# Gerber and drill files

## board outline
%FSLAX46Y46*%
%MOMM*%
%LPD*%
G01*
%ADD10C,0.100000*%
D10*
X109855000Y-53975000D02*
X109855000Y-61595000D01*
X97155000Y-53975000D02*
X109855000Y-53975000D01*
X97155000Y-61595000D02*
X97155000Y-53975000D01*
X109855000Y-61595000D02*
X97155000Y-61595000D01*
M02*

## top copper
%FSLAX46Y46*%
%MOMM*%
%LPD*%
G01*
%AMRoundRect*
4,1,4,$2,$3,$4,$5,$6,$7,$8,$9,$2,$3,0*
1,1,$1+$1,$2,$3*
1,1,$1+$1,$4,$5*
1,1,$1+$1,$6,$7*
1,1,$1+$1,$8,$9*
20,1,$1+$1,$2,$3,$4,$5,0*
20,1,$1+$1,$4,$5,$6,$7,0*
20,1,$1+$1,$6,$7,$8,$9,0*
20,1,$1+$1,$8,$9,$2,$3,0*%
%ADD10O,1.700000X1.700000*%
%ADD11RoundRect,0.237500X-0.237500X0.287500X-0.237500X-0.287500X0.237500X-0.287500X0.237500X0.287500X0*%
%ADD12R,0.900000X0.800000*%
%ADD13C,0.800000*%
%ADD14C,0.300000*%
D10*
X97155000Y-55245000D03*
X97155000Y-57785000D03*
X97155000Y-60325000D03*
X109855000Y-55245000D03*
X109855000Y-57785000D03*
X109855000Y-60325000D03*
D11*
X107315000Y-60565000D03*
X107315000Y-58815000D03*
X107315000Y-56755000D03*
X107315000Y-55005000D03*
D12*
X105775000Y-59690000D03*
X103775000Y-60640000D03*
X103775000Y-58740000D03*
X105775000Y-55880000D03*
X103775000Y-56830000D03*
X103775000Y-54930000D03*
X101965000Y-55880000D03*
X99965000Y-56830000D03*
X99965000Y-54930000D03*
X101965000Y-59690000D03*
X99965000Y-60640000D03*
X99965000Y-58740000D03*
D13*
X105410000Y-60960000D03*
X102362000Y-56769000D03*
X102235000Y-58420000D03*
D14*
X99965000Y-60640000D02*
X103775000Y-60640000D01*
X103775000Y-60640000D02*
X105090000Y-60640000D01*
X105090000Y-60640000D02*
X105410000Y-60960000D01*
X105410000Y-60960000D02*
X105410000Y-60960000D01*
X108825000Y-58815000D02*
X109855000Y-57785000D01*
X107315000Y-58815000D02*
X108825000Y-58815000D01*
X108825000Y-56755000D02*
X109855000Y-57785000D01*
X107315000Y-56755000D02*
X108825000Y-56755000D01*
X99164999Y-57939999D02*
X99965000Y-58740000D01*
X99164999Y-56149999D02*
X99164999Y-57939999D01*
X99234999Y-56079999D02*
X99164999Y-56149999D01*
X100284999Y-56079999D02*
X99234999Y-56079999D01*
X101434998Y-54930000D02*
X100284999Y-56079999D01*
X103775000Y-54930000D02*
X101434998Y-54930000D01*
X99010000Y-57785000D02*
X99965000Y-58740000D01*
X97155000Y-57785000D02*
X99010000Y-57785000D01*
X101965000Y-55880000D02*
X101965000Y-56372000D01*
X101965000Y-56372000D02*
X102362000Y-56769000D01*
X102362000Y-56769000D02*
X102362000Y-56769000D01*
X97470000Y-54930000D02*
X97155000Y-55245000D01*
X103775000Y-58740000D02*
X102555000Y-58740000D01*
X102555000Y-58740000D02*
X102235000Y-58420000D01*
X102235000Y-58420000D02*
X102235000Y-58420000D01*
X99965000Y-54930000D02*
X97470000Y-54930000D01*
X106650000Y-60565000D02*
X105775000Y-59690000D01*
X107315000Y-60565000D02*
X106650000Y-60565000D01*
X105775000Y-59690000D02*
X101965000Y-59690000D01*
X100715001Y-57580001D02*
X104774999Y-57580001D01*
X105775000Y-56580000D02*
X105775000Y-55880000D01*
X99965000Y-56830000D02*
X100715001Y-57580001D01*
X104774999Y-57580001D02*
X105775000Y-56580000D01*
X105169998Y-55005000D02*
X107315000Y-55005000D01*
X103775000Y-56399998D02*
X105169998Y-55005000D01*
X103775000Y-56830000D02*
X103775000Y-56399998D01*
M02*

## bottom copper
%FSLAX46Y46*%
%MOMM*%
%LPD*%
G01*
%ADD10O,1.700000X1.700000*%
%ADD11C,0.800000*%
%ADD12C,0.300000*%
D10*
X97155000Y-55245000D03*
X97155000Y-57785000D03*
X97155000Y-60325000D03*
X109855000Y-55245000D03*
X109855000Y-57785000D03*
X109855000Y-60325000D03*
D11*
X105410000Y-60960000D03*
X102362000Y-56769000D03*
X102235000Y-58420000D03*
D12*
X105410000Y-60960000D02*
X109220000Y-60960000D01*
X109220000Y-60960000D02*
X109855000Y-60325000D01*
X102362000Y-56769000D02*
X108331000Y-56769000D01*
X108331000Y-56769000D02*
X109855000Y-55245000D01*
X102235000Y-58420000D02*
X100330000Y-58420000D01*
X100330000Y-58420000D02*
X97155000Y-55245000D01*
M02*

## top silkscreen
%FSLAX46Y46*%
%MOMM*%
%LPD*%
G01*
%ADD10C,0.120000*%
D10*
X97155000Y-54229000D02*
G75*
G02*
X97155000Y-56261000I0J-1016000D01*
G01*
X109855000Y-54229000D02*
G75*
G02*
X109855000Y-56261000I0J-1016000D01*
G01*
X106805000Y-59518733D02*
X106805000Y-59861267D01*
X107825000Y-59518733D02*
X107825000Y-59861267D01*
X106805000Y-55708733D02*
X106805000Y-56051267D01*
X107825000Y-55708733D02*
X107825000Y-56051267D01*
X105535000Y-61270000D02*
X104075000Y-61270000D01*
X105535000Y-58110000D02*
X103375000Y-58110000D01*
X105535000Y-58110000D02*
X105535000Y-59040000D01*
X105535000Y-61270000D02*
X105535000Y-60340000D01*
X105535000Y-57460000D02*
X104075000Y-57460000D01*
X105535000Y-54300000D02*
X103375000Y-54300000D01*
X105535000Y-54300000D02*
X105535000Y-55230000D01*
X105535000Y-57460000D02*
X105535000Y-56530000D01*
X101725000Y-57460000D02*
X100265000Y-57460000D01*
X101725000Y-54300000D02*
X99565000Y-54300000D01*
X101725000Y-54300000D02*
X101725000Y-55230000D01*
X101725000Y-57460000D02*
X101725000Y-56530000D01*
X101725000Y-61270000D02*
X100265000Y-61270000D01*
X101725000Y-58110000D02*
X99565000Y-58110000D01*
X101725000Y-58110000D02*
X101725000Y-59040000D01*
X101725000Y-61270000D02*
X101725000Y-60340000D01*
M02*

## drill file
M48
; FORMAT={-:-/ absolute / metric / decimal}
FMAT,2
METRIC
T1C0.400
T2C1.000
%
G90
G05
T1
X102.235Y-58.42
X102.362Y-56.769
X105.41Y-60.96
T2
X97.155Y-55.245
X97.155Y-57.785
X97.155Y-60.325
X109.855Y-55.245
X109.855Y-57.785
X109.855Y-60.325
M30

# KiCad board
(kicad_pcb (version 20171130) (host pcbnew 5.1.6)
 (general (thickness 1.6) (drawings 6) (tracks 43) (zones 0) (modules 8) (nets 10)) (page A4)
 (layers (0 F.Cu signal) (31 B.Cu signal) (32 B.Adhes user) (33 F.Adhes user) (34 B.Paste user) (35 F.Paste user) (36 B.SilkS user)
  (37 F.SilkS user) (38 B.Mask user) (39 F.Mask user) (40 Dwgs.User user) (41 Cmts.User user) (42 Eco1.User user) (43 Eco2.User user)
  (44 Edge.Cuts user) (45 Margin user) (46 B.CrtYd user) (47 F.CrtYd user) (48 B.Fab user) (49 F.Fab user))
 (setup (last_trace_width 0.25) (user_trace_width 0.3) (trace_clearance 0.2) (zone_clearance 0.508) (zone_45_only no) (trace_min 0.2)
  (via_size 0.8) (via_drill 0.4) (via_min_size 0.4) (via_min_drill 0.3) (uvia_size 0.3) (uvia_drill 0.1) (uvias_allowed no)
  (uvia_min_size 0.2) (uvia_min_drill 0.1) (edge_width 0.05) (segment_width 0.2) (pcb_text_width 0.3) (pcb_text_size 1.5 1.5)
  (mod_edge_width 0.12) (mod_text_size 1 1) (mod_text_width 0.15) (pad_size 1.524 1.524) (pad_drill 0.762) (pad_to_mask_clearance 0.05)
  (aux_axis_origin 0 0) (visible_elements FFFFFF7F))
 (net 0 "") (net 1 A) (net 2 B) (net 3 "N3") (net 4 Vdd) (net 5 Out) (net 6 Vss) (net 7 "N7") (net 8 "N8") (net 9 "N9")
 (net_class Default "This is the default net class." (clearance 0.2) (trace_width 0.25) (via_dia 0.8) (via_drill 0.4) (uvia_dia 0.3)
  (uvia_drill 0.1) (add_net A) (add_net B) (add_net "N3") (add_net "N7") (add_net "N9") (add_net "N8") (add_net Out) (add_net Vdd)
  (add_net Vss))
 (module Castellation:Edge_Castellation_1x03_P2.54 (layer F.Cu) (at 97.155 55.245)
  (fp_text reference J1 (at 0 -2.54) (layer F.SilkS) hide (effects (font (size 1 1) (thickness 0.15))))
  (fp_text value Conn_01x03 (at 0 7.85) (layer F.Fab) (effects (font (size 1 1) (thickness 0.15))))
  (fp_arc (start 0 0) (end 0 1.016) (angle -180) (layer F.SilkS) (width 0.12))
  (pad 1 thru_hole oval (at 0 0) (size 1.7 1.7) (drill 1) (layers *.Cu *.Mask) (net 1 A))
  (pad 2 thru_hole oval (at 0 2.54) (size 1.7 1.7) (drill 1) (layers *.Cu *.Mask) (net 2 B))
  (pad 3 thru_hole oval (at 0 5.08) (size 1.7 1.7) (drill 1) (layers *.Cu *.Mask) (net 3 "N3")))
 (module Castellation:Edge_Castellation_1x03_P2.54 (layer F.Cu) (at 109.855 55.245)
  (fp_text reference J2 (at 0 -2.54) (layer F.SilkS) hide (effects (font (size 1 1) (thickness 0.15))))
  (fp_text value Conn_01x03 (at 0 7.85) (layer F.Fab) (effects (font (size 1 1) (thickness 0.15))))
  (fp_arc (start 0 0) (end 0 1.016) (angle -180) (layer F.SilkS) (width 0.12))
  (pad 1 thru_hole oval (at 0 0) (size 1.7 1.7) (drill 1) (layers *.Cu *.Mask) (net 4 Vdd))
  (pad 2 thru_hole oval (at 0 2.54) (size 1.7 1.7) (drill 1) (layers *.Cu *.Mask) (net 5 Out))
  (pad 3 thru_hole oval (at 0 5.08) (size 1.7 1.7) (drill 1) (layers *.Cu *.Mask) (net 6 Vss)))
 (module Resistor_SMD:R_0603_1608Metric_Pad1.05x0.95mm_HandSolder (layer F.Cu) (at 107.315 59.69 270)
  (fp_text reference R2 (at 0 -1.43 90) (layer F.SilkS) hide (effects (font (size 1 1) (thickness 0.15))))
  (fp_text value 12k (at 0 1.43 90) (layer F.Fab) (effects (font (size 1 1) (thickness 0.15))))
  (fp_line (start -0.171267 0.51) (end 0.171267 0.51) (layer F.SilkS) (width 0.12))
  (fp_line (start -0.171267 -0.51) (end 0.171267 -0.51) (layer F.SilkS) (width 0.12))
  (pad 2 smd roundrect (at 0.875 0 270) (size 1.05 0.95) (layers F.Cu F.Paste F.Mask) (roundrect_rratio 0.25) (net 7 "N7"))
  (pad 1 smd roundrect (at -0.875 0 270) (size 1.05 0.95) (layers F.Cu F.Paste F.Mask) (roundrect_rratio 0.25) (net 5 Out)))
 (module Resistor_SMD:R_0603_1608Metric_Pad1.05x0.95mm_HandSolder (layer F.Cu) (at 107.315 55.88 270)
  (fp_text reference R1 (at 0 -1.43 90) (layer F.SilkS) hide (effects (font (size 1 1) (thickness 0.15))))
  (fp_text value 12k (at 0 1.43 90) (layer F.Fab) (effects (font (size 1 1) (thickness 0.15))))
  (fp_line (start -0.171267 0.51) (end 0.171267 0.51) (layer F.SilkS) (width 0.12))
  (fp_line (start -0.171267 -0.51) (end 0.171267 -0.51) (layer F.SilkS) (width 0.12))
  (pad 2 smd roundrect (at 0.875 0 270) (size 1.05 0.95) (layers F.Cu F.Paste F.Mask) (roundrect_rratio 0.25) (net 5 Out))
  (pad 1 smd roundrect (at -0.875 0 270) (size 1.05 0.95) (layers F.Cu F.Paste F.Mask) (roundrect_rratio 0.25) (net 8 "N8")))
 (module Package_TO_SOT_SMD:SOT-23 (layer F.Cu) (at 104.775 59.69)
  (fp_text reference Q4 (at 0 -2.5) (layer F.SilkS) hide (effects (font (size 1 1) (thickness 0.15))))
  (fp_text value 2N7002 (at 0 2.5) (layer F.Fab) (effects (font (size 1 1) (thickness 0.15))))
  (fp_line (start 0.76 1.58) (end -0.7 1.58) (layer F.SilkS) (width 0.12))
  (fp_line (start 0.76 -1.58) (end -1.4 -1.58) (layer F.SilkS) (width 0.12))
  (fp_line (start 0.76 -1.58) (end 0.76 -0.65) (layer F.SilkS) (width 0.12))
  (fp_line (start 0.76 1.58) (end 0.76 0.65) (layer F.SilkS) (width 0.12))
  (pad 3 smd rect (at 1 0) (size 0.9 0.8) (layers F.Cu F.Paste F.Mask) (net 7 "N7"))
  (pad 2 smd rect (at -1 0.95) (size 0.9 0.8) (layers F.Cu F.Paste F.Mask) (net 6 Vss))
  (pad 1 smd rect (at -1 -0.95) (size 0.9 0.8) (layers F.Cu F.Paste F.Mask) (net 1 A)))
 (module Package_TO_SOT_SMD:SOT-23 (layer F.Cu) (at 104.775 55.88)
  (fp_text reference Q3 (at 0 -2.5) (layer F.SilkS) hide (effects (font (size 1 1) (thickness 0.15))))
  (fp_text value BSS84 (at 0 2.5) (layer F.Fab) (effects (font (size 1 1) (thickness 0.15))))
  (fp_line (start 0.76 1.58) (end -0.7 1.58) (layer F.SilkS) (width 0.12))
  (fp_line (start 0.76 -1.58) (end -1.4 -1.58) (layer F.SilkS) (width 0.12))
  (fp_line (start 0.76 -1.58) (end 0.76 -0.65) (layer F.SilkS) (width 0.12))
  (fp_line (start 0.76 1.58) (end 0.76 0.65) (layer F.SilkS) (width 0.12))
  (pad 3 smd rect (at 1 0) (size 0.9 0.8) (layers F.Cu F.Paste F.Mask) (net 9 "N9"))
  (pad 2 smd rect (at -1 0.95) (size 0.9 0.8) (layers F.Cu F.Paste F.Mask) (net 8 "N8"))
  (pad 1 smd rect (at -1 -0.95) (size 0.9 0.8) (layers F.Cu F.Paste F.Mask) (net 2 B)))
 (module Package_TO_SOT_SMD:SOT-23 (layer F.Cu) (at 100.965 55.88)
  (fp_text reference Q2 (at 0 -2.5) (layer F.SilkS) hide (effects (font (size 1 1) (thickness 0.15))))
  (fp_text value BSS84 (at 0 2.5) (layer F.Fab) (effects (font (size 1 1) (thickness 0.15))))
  (fp_line (start 0.76 1.58) (end -0.7 1.58) (layer F.SilkS) (width 0.12))
  (fp_line (start 0.76 -1.58) (end -1.4 -1.58) (layer F.SilkS) (width 0.12))
  (fp_line (start 0.76 -1.58) (end 0.76 -0.65) (layer F.SilkS) (width 0.12))
  (fp_line (start 0.76 1.58) (end 0.76 0.65) (layer F.SilkS) (width 0.12))
  (pad 3 smd rect (at 1 0) (size 0.9 0.8) (layers F.Cu F.Paste F.Mask) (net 4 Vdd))
  (pad 2 smd rect (at -1 0.95) (size 0.9 0.8) (layers F.Cu F.Paste F.Mask) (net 9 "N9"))
  (pad 1 smd rect (at -1 -0.95) (size 0.9 0.8) (layers F.Cu F.Paste F.Mask) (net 1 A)))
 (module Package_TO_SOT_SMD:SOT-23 (layer F.Cu) (at 100.965 59.69)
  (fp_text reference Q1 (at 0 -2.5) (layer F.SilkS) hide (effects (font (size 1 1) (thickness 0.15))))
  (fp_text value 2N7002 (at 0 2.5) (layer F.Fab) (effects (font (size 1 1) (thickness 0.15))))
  (fp_line (start 0.76 1.58) (end -0.7 1.58) (layer F.SilkS) (width 0.12))
  (fp_line (start 0.76 -1.58) (end -1.4 -1.58) (layer F.SilkS) (width 0.12))
  (fp_line (start 0.76 -1.58) (end 0.76 -0.65) (layer F.SilkS) (width 0.12))
  (fp_line (start 0.76 1.58) (end 0.76 0.65) (layer F.SilkS) (width 0.12))
  (pad 3 smd rect (at 1 0) (size 0.9 0.8) (layers F.Cu F.Paste F.Mask) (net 7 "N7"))
  (pad 2 smd rect (at -1 0.95) (size 0.9 0.8) (layers F.Cu F.Paste F.Mask) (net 6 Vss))
  (pad 1 smd rect (at -1 -0.95) (size 0.9 0.8) (layers F.Cu F.Paste F.Mask) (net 2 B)))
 (gr_line (start 109.855 53.975) (end 109.855 61.595) (layer Edge.Cuts) (width 0.1))
 (gr_line (start 97.155 53.975) (end 109.855 53.975) (layer Edge.Cuts) (width 0.1))
 (gr_line (start 97.155 61.595) (end 97.155 53.975) (layer Edge.Cuts) (width 0.1))
 (gr_line (start 109.855 61.595) (end 97.155 61.595) (layer Edge.Cuts) (width 0.1))
 (segment (start 99.965 60.64) (end 103.775 60.64) (width 0.3) (layer F.Cu) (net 6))
 (segment (start 103.775 60.64) (end 105.09 60.64) (width 0.3) (layer F.Cu) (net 6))
 (segment (start 105.09 60.64) (end 105.41 60.96) (width 0.3) (layer F.Cu) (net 6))
 (segment (start 105.41 60.96) (end 105.41 60.96) (width 0.3) (layer F.Cu) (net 6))
 (via (at 105.41 60.96) (size 0.8) (drill 0.4) (layers F.Cu B.Cu) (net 6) (status 1000000))
 (segment (start 105.41 60.96) (end 109.22 60.96) (width 0.3) (layer B.Cu) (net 6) (status 1000000))
 (segment (start 109.22 60.96) (end 109.855 60.325) (width 0.3) (layer B.Cu) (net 6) (status 1000000))
 (segment (start 108.825 58.815) (end 109.855 57.785) (width 0.3) (layer F.Cu) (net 5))
 (segment (start 107.315 58.815) (end 108.825 58.815) (width 0.3) (layer F.Cu) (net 5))
 (segment (start 108.825 56.755) (end 109.855 57.785) (width 0.3) (layer F.Cu) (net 5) (status 1000000))
 (segment (start 107.315 56.755) (end 108.825 56.755) (width 0.3) (layer F.Cu) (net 5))
 (segment (start 99.164999 57.939999) (end 99.965 58.74) (width 0.3) (layer F.Cu) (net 2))
 (segment (start 99.164999 56.149999) (end 99.164999 57.939999) (width 0.3) (layer F.Cu) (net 2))
 (segment (start 99.234999 56.079999) (end 99.164999 56.149999) (width 0.3) (layer F.Cu) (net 2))
 (segment (start 100.284999 56.079999) (end 99.234999 56.079999) (width 0.3) (layer F.Cu) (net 2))
 (segment (start 101.434998 54.93) (end 100.284999 56.079999) (width 0.3) (layer F.Cu) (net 2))
 (segment (start 103.775 54.93) (end 101.434998 54.93) (width 0.3) (layer F.Cu) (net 2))
 (segment (start 99.01 57.785) (end 99.965 58.74) (width 0.3) (layer F.Cu) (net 2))
 (segment (start 97.155 57.785) (end 99.01 57.785) (width 0.3) (layer F.Cu) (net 2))
 (segment (start 101.965 55.88) (end 101.965 56.372) (width 0.3) (layer F.Cu) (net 4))
 (segment (start 101.965 56.372) (end 102.362 56.769) (width 0.3) (layer F.Cu) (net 4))
 (segment (start 102.362 56.769) (end 102.362 56.769) (width 0.3) (layer F.Cu) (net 4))
 (via (at 102.362 56.769) (size 0.8) (drill 0.4) (layers F.Cu B.Cu) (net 4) (status 1000000))
 (segment (start 102.362 56.769) (end 108.331 56.769) (width 0.3) (layer B.Cu) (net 4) (status 1000000))
 (segment (start 108.331 56.769) (end 109.855 55.245) (width 0.3) (layer B.Cu) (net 4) (status 1000000))
 (segment (start 97.47 54.93) (end 97.155 55.245) (width 0.3) (layer F.Cu) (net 1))
 (segment (start 103.775 58.74) (end 102.555 58.74) (width 0.3) (layer F.Cu) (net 1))
 (segment (start 102.555 58.74) (end 102.235 58.42) (width 0.3) (layer F.Cu) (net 1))
 (segment (start 102.235 58.42) (end 102.235 58.42) (width 0.3) (layer F.Cu) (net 1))
 (segment (start 99.965 54.93) (end 97.47 54.93) (width 0.3) (layer F.Cu) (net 1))
 (segment (start 102.235 58.42) (end 100.33 58.42) (width 0.3) (layer B.Cu) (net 1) (status 1000000))
 (via (at 102.235 58.42) (size 0.8) (drill 0.4) (layers F.Cu B.Cu) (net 1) (status 1000000))
 (segment (start 100.33 58.42) (end 97.155 55.245) (width 0.3) (layer B.Cu) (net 1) (status 1000000))
 (segment (start 106.65 60.565) (end 105.775 59.69) (width 0.3) (layer F.Cu) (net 7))
 (segment (start 107.315 60.565) (end 106.65 60.565) (width 0.3) (layer F.Cu) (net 7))
 (segment (start 105.775 59.69) (end 101.965 59.69) (width 0.3) (layer F.Cu) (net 7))
 (segment (start 100.715001 57.580001) (end 104.774999 57.580001) (width 0.3) (layer F.Cu) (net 9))
 (segment (start 105.775 56.58) (end 105.775 55.88) (width 0.3) (layer F.Cu) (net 9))
 (segment (start 99.965 56.83) (end 100.715001 57.580001) (width 0.3) (layer F.Cu) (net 9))
 (segment (start 104.774999 57.580001) (end 105.775 56.58) (width 0.3) (layer F.Cu) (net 9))
 (segment (start 105.169998 55.005) (end 107.315 55.005) (width 0.3) (layer F.Cu) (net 8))
 (segment (start 103.775 56.399998) (end 105.169998 55.005) (width 0.3) (layer F.Cu) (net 8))
 (segment (start 103.775 56.83) (end 103.775 56.399998) (width 0.3) (layer F.Cu) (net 8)))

